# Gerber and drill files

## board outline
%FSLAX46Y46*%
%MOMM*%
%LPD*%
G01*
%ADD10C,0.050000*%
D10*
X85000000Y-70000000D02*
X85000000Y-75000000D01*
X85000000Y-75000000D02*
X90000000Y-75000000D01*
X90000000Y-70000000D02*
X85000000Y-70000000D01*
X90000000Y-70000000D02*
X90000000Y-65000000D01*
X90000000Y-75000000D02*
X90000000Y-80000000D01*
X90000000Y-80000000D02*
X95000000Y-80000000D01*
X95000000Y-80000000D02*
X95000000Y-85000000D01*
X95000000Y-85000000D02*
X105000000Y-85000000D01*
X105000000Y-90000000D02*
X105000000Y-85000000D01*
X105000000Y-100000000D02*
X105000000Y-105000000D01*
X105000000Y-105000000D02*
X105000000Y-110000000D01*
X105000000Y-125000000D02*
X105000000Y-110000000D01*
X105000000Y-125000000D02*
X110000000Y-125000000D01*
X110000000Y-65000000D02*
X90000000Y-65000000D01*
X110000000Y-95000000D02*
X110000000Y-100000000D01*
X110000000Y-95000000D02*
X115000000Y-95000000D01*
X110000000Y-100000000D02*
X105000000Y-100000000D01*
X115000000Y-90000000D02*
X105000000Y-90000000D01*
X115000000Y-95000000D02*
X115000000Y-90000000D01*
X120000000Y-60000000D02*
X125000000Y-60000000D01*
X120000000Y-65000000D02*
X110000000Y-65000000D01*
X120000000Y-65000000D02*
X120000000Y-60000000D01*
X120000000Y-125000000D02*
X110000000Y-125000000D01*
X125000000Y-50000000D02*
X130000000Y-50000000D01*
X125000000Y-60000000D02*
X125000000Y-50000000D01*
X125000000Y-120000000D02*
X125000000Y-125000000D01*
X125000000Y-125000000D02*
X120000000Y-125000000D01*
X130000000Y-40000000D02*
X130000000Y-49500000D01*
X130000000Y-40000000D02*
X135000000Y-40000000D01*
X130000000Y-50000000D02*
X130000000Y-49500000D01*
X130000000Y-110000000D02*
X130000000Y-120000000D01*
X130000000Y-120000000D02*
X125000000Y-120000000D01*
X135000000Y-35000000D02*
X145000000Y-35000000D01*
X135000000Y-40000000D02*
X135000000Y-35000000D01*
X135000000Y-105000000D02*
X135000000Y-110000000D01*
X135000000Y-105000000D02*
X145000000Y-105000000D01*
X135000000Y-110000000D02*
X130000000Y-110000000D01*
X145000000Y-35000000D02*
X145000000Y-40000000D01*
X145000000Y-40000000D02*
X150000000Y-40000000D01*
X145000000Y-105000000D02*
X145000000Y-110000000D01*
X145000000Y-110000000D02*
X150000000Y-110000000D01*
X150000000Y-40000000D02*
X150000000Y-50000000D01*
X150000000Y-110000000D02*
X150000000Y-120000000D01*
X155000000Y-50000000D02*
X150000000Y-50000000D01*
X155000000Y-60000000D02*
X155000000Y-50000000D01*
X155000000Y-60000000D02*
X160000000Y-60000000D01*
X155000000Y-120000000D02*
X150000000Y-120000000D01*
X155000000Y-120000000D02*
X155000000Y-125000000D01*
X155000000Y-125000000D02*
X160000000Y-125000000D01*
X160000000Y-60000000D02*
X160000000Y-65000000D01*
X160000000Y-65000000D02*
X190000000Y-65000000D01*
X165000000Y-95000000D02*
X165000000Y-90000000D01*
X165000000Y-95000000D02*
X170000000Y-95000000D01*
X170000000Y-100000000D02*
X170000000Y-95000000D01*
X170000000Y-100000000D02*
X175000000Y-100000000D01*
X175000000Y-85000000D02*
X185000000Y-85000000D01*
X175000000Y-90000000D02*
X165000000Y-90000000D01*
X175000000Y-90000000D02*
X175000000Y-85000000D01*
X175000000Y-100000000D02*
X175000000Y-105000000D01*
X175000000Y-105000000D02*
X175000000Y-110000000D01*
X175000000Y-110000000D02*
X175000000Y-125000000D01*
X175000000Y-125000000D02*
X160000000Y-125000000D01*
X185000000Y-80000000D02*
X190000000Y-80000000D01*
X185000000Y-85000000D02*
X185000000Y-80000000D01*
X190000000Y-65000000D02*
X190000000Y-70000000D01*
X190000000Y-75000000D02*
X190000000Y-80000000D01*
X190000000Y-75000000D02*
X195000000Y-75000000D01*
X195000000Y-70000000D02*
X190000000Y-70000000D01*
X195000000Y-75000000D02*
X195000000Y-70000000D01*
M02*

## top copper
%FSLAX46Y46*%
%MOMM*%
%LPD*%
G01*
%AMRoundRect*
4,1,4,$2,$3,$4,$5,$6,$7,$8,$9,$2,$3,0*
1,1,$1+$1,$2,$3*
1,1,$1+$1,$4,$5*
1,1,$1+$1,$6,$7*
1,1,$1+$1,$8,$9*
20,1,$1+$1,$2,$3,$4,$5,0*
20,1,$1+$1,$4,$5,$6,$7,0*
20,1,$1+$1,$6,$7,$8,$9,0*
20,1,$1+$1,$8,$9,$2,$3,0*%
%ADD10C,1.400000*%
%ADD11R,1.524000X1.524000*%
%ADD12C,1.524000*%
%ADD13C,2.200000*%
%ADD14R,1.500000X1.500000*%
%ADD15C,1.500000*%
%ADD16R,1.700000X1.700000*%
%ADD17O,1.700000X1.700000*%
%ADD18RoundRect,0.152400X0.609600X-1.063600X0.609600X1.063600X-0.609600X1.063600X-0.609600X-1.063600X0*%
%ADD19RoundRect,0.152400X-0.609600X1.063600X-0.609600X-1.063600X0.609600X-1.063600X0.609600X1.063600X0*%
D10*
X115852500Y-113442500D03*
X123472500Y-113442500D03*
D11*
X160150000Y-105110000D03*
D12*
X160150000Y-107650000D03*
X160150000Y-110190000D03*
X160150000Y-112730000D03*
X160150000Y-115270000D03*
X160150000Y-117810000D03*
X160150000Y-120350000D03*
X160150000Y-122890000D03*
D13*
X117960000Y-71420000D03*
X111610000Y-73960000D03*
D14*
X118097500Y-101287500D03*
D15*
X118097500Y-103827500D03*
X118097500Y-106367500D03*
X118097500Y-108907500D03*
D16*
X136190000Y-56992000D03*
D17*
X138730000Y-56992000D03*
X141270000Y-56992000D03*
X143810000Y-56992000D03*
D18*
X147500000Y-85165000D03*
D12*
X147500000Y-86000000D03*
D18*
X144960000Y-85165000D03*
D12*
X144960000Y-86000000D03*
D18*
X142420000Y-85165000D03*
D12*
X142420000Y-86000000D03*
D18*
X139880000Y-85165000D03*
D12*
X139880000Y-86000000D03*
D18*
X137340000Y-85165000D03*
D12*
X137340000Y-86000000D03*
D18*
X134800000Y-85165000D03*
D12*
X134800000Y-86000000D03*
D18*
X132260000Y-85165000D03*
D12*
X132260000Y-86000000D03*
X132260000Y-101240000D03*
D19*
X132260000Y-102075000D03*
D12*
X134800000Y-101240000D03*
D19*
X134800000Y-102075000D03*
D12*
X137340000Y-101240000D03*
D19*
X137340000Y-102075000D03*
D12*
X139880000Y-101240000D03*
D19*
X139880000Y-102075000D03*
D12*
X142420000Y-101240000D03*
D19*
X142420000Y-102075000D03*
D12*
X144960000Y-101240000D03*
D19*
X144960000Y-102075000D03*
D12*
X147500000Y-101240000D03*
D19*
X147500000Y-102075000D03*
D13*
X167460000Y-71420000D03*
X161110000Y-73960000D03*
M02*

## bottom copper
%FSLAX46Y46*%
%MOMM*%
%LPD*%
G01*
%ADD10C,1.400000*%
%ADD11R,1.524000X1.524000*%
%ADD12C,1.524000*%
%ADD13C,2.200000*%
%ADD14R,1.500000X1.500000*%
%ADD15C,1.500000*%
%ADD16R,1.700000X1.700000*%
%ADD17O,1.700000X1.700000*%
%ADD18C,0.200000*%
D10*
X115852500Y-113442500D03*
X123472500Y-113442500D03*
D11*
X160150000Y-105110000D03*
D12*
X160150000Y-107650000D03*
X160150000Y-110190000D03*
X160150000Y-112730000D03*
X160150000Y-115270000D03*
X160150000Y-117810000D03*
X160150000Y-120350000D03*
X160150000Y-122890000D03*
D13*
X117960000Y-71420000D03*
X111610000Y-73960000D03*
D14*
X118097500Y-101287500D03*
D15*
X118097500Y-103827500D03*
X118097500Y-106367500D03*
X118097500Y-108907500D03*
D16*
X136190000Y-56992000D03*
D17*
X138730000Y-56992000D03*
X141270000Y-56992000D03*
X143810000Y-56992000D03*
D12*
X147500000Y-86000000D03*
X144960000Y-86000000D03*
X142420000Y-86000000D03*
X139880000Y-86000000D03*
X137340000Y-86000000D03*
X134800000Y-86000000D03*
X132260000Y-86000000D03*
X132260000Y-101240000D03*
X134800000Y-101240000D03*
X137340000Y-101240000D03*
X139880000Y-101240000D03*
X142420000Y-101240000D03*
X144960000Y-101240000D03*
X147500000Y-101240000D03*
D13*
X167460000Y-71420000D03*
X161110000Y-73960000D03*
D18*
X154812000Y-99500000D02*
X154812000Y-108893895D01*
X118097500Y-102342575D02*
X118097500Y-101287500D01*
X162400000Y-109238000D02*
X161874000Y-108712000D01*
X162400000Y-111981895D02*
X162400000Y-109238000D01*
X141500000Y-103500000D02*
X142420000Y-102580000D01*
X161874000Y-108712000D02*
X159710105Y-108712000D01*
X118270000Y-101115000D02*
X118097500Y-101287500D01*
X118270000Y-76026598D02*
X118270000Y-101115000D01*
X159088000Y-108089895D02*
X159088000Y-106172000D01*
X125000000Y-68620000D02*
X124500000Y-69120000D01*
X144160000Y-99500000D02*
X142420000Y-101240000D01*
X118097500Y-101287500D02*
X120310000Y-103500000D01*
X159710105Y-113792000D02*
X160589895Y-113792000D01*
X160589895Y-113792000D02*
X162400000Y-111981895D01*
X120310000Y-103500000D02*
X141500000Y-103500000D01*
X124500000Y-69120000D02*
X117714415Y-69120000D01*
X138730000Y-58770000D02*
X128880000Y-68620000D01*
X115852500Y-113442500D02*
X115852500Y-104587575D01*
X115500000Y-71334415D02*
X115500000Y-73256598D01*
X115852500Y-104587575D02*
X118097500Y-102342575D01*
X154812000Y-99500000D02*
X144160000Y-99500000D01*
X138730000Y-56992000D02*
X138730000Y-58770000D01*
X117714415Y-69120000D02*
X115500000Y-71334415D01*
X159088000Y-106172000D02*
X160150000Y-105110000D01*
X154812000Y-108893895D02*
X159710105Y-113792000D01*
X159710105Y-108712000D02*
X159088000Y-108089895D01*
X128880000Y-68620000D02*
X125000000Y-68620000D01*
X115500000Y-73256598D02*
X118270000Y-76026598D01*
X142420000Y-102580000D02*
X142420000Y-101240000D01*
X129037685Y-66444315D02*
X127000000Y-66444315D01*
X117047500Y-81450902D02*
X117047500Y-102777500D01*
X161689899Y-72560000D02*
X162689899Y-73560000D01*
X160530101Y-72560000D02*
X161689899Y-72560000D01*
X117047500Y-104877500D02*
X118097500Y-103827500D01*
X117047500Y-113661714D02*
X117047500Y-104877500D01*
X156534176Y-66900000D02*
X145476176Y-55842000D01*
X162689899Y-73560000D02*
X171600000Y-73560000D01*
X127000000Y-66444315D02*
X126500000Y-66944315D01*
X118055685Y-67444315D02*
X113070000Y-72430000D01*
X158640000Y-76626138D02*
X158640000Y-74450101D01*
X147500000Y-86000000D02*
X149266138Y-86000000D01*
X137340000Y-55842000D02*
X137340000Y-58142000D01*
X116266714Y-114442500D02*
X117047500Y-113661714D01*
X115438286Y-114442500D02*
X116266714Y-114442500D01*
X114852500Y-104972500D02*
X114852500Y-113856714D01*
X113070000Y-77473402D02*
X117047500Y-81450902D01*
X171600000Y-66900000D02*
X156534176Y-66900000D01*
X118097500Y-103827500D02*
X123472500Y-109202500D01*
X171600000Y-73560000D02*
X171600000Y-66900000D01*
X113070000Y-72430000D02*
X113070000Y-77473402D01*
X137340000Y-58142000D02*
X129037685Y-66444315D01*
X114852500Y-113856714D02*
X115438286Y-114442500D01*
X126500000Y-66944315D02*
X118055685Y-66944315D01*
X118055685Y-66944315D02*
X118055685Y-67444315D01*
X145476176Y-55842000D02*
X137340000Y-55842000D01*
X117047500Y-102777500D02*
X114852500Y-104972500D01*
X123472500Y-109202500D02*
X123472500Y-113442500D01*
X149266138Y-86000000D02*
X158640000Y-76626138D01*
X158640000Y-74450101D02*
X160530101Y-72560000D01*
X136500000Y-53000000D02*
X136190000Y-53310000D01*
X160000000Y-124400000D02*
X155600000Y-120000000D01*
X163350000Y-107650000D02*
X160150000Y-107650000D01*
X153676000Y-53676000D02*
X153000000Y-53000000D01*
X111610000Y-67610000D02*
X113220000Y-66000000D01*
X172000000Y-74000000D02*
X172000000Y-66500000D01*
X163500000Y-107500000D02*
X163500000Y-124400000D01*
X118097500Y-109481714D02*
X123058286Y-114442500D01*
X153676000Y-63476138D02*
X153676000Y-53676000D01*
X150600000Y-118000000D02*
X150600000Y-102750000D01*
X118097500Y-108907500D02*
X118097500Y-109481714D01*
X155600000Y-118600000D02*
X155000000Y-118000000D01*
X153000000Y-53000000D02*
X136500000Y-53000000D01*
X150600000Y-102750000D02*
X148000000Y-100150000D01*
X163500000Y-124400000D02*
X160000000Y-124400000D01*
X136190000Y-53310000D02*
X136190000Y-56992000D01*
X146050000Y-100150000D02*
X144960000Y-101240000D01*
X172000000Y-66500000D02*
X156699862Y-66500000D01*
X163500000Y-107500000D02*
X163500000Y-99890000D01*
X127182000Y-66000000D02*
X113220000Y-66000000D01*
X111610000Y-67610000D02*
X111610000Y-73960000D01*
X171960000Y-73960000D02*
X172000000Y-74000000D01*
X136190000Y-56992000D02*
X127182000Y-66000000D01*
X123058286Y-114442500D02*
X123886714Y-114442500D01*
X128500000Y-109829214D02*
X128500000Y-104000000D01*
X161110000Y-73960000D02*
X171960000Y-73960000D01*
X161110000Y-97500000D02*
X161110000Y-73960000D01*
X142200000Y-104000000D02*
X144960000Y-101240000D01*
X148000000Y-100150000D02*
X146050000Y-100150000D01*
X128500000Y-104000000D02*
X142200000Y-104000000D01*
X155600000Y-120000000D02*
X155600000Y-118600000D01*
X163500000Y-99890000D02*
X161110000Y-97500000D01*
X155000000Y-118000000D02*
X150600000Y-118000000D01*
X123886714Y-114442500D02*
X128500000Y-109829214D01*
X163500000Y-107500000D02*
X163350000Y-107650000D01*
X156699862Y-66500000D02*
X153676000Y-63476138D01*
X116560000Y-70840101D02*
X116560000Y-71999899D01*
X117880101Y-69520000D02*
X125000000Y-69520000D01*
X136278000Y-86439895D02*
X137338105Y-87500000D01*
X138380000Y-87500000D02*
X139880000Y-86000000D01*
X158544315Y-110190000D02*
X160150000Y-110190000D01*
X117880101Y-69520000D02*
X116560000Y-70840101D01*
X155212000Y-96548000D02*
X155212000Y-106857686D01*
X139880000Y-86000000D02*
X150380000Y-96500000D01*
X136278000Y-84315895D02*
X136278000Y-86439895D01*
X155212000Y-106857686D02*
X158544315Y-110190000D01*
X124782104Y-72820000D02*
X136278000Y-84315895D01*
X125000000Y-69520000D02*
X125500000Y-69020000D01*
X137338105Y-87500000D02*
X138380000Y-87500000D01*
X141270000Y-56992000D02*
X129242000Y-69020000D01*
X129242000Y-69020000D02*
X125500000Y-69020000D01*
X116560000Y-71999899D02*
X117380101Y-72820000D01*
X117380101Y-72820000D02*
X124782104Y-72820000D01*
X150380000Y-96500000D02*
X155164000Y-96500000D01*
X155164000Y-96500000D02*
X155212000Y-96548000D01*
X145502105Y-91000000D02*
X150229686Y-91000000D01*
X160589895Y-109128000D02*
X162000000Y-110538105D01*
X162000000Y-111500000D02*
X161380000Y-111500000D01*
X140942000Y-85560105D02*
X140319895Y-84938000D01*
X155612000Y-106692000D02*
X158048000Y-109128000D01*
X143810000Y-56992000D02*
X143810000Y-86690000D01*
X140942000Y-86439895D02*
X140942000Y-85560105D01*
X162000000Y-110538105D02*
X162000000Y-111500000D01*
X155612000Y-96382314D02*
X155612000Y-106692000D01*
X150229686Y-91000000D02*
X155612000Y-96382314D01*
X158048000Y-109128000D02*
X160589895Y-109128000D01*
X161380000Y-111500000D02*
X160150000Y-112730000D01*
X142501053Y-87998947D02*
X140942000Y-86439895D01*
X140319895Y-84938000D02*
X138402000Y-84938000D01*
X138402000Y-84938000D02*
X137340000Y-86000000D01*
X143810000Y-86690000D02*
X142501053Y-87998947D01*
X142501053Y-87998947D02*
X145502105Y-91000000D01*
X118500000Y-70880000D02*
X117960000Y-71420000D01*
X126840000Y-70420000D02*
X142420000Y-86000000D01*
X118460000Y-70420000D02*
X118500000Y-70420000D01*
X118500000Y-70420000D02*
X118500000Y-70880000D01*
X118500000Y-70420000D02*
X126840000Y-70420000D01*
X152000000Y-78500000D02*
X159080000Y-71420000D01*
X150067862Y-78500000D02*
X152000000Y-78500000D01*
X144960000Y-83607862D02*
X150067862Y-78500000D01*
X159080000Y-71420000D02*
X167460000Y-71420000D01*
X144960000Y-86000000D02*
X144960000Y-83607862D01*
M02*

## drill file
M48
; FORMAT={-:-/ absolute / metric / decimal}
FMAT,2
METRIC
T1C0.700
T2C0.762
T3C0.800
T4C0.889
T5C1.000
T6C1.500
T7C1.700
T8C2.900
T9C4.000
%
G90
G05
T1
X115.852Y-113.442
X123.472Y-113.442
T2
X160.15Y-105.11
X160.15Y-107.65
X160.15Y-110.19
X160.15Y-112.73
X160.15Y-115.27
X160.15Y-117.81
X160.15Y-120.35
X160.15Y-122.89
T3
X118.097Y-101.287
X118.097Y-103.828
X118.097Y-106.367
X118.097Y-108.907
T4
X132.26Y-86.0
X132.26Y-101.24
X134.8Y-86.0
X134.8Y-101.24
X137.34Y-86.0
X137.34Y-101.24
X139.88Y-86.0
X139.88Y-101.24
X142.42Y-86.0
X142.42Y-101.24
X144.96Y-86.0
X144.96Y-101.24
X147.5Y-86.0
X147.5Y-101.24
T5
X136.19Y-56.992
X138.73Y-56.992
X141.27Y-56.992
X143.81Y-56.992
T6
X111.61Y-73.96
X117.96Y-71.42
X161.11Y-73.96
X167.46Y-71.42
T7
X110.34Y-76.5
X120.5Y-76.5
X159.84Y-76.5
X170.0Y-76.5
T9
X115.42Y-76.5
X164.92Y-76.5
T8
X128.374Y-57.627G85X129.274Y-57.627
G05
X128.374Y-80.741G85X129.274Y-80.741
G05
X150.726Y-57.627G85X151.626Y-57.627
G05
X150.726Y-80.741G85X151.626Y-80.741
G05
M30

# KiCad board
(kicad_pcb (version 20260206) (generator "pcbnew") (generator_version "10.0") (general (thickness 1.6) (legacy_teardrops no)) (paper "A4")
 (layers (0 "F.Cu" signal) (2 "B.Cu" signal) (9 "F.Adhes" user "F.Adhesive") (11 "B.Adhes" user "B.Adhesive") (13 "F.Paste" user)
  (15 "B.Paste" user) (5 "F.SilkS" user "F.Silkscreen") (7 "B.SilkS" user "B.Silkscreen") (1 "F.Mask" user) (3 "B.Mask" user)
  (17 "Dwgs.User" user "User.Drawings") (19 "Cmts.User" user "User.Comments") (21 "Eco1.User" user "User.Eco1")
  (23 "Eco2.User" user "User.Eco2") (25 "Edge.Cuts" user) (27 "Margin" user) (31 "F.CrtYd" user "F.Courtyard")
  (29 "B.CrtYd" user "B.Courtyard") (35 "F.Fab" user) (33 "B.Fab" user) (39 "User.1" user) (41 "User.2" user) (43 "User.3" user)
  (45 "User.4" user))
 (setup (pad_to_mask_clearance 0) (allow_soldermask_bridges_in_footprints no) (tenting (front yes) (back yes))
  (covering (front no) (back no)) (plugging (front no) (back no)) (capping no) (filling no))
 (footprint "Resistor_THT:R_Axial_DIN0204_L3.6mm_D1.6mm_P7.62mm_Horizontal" (layer "F.Cu") (at 115.8525 113.4425)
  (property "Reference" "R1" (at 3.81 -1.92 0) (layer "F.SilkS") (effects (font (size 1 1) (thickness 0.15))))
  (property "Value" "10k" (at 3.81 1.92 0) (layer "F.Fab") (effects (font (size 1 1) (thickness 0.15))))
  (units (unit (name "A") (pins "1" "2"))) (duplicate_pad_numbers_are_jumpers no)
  (pad "1" thru_hole circle (at 0 0) (size 1.4 1.4) (drill 0.7) (layers "*.Cu" "*.Mask") (remove_unused_layers no) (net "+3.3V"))
  (pad "2" thru_hole circle (at 7.62 0) (size 1.4 1.4) (drill 0.7) (layers "*.Cu" "*.Mask") (remove_unused_layers no) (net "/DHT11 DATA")))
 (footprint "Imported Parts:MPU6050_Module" (layer "F.Cu") (at 160.15 105.11)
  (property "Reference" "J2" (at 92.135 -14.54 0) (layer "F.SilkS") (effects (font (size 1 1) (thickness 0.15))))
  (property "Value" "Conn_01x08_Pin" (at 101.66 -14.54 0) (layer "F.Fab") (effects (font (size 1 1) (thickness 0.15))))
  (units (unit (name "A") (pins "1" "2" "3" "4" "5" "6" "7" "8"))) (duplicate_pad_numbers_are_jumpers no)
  (pad "1" thru_hole rect (at 0 0) (size 1.524 1.524) (drill 0.762) (layers "*.Cu" "*.Mask") (remove_unused_layers no) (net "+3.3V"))
  (pad "2" thru_hole circle (at 0 2.54) (size 1.524 1.524) (drill 0.762) (layers "*.Cu" "*.Mask") (remove_unused_layers no) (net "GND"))
  (pad "3" thru_hole circle (at 0 5.08) (size 1.524 1.524) (drill 0.762) (layers "*.Cu" "*.Mask") (remove_unused_layers no) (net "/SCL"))
  (pad "4" thru_hole circle (at 0 7.62) (size 1.524 1.524) (drill 0.762) (layers "*.Cu" "*.Mask") (remove_unused_layers no) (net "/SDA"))
  (pad "5" thru_hole circle (at 0 10.16) (size 1.524 1.524) (drill 0.762) (layers "*.Cu" "*.Mask") (remove_unused_layers no)
   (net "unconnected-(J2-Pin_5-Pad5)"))
  (pad "6" thru_hole circle (at 0 12.7) (size 1.524 1.524) (drill 0.762) (layers "*.Cu" "*.Mask") (remove_unused_layers no)
   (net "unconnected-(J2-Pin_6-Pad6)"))
  (pad "7" thru_hole circle (at 0 15.24) (size 1.524 1.524) (drill 0.762) (layers "*.Cu" "*.Mask") (remove_unused_layers no)
   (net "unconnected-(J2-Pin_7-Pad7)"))
  (pad "8" thru_hole circle (at 0 17.78) (size 1.524 1.524) (drill 0.762) (layers "*.Cu" "*.Mask") (remove_unused_layers no)
   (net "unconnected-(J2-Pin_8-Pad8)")))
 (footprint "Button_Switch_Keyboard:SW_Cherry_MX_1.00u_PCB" (layer "F.Cu") (at 117.96 71.42)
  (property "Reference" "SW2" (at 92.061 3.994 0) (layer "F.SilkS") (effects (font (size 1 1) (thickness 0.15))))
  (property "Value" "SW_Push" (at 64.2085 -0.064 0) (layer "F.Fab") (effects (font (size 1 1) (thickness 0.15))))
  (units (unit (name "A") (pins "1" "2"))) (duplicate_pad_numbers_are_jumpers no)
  (pad "" np_thru_hole circle (at -7.62 5.08) (size 1.7 1.7) (drill 1.7) (layers "*.Cu" "*.Mask"))
  (pad "" np_thru_hole circle (at -2.54 5.08) (size 4 4) (drill 4) (layers "*.Cu" "*.Mask"))
  (pad "" np_thru_hole circle (at 2.54 5.08) (size 1.7 1.7) (drill 1.7) (layers "*.Cu" "*.Mask"))
  (pad "1" thru_hole circle (at 0 0) (size 2.2 2.2) (drill 1.5) (layers "*.Cu" "*.Mask") (remove_unused_layers no) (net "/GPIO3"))
  (pad "2" thru_hole circle (at -6.35 2.54) (size 2.2 2.2) (drill 1.5) (layers "*.Cu" "*.Mask") (remove_unused_layers no) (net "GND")))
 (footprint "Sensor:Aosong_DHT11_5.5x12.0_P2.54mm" (layer "F.Cu") (at 118.0975 101.2875)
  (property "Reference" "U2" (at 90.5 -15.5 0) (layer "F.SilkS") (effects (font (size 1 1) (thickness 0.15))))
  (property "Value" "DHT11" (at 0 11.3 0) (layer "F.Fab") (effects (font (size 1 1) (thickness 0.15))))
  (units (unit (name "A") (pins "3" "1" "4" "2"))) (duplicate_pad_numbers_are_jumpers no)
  (pad "1" thru_hole rect (at 0 0) (size 1.5 1.5) (drill 0.8) (layers "*.Cu" "*.Mask") (remove_unused_layers no) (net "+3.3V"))
  (pad "2" thru_hole circle (at 0 2.54) (size 1.5 1.5) (drill 0.8) (layers "*.Cu" "*.Mask") (remove_unused_layers no) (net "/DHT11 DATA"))
  (pad "3" thru_hole circle (at 0 5.08) (size 1.5 1.5) (drill 0.8) (layers "*.Cu" "*.Mask") (remove_unused_layers no)
   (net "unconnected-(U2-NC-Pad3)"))
  (pad "4" thru_hole circle (at 0 7.62) (size 1.5 1.5) (drill 0.8) (layers "*.Cu" "*.Mask") (remove_unused_layers no) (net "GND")))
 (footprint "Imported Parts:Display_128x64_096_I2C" (layer "F.Cu") (at 140 56.992)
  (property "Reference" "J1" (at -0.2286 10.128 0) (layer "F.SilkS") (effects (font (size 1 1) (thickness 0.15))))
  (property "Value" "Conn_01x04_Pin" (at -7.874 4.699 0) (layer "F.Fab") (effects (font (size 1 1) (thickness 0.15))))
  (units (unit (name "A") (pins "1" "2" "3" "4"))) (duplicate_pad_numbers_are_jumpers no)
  (pad "" np_thru_hole oval (at -11.176 0.635) (size 3.8 2.9) (drill oval 3.8 2.9) (layers "*.Cu" "*.Mask"))
  (pad "" np_thru_hole oval (at -11.176 23.749) (size 3.8 2.9) (drill oval 3.8 2.9) (layers "*.Cu" "*.Mask"))
  (pad "" np_thru_hole oval (at 11.176 0.635) (size 3.8 2.9) (drill oval 3.8 2.9) (layers "*.Cu" "*.Mask"))
  (pad "" np_thru_hole oval (at 11.176 23.749) (size 3.8 2.9) (drill oval 3.8 2.9) (layers "*.Cu" "*.Mask"))
  (pad "1" thru_hole rect (at -3.81 0 90) (size 1.7 1.7) (drill 1) (layers "*.Cu" "*.Mask") (remove_unused_layers no) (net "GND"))
  (pad "2" thru_hole oval (at -1.27 0 90) (size 1.7 1.7) (drill 1) (layers "*.Cu" "*.Mask") (remove_unused_layers no) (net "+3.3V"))
  (pad "3" thru_hole oval (at 1.27 0 90) (size 1.7 1.7) (drill 1) (layers "*.Cu" "*.Mask") (remove_unused_layers no) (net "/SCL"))
  (pad "4" thru_hole oval (at 3.81 0 90) (size 1.7 1.7) (drill 1) (layers "*.Cu" "*.Mask") (remove_unused_layers no) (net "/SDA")))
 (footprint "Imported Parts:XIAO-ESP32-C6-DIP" (layer "F.Cu") (at 139.88 93.62)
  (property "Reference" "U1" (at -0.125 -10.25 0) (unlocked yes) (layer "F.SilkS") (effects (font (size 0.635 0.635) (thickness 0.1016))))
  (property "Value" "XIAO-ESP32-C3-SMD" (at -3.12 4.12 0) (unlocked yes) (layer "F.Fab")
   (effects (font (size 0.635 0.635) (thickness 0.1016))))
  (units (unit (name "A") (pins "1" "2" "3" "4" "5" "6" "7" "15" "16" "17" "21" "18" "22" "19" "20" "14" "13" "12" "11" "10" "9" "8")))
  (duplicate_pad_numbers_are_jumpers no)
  (pad "1" smd roundrect (at 7.62 -8.455 90) (size 2.432 1.524) (layers "F.Cu" "F.Mask") (roundrect_rratio 0.1) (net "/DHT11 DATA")
   (thermal_bridge_angle 45))
  (pad "1" thru_hole circle (at 7.62 -7.62 90) (size 1.524 1.524) (drill 0.889) (layers "*.Cu" "*.Mask") (remove_unused_layers no)
   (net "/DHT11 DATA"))
  (pad "2" smd roundrect (at 5.08 -8.455 90) (size 2.432 1.524) (layers "F.Cu" "F.Mask") (roundrect_rratio 0.1) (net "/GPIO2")
   (thermal_bridge_angle 45))
  (pad "2" thru_hole circle (at 5.08 -7.62 90) (size 1.524 1.524) (drill 0.889) (layers "*.Cu" "*.Mask") (remove_unused_layers no)
   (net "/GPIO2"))
  (pad "3" smd roundrect (at 2.54 -8.455 90) (size 2.432 1.524) (layers "F.Cu" "F.Mask") (roundrect_rratio 0.1) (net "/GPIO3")
   (thermal_bridge_angle 45))
  (pad "3" thru_hole circle (at 2.54 -7.62 90) (size 1.524 1.524) (drill 0.889) (layers "*.Cu" "*.Mask") (remove_unused_layers no)
   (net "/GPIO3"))
  (pad "4" smd roundrect (at 0 -8.455 90) (size 2.432 1.524) (layers "F.Cu" "F.Mask") (roundrect_rratio 0.1) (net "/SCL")
   (thermal_bridge_angle 45))
  (pad "4" thru_hole circle (at 0 -7.62 90) (size 1.524 1.524) (drill 0.889) (layers "*.Cu" "*.Mask") (remove_unused_layers no) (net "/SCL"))
  (pad "5" smd roundrect (at -2.54 -8.455 90) (size 2.432 1.524) (layers "F.Cu" "F.Mask") (roundrect_rratio 0.1) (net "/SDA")
   (thermal_bridge_angle 45))
  (pad "5" thru_hole circle (at -2.54 -7.62 90) (size 1.524 1.524) (drill 0.889) (layers "*.Cu" "*.Mask") (remove_unused_layers no)
   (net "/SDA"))
  (pad "6" smd roundrect (at -5.08 -8.455 90) (size 2.432 1.524) (layers "F.Cu" "F.Mask") (roundrect_rratio 0.1)
   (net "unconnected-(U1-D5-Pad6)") (thermal_bridge_angle 45))
  (pad "6" thru_hole circle (at -5.08 -7.62 90) (size 1.524 1.524) (drill 0.889) (layers "*.Cu" "*.Mask") (remove_unused_layers no)
   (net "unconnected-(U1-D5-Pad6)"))
  (pad "7" smd roundrect (at -7.62 -8.455 90) (size 2.432 1.524) (layers "F.Cu" "F.Mask") (roundrect_rratio 0.1)
   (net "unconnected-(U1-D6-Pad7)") (thermal_bridge_angle 45))
  (pad "7" thru_hole circle (at -7.62 -7.62 90) (size 1.524 1.524) (drill 0.889) (layers "*.Cu" "*.Mask") (remove_unused_layers no)
   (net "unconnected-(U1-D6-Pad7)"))
  (pad "8" thru_hole circle (at -7.62 7.62 270) (size 1.524 1.524) (drill 0.889) (layers "*.Cu" "*.Mask") (remove_unused_layers no)
   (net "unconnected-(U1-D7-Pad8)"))
  (pad "8" smd roundrect (at -7.62 8.455 270) (size 2.432 1.524) (layers "F.Cu" "F.Mask") (roundrect_rratio 0.1)
   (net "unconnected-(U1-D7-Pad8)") (thermal_bridge_angle 45))
  (pad "9" thru_hole circle (at -5.08 7.62 270) (size 1.524 1.524) (drill 0.889) (layers "*.Cu" "*.Mask") (remove_unused_layers no)
   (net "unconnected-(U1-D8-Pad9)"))
  (pad "9" smd roundrect (at -5.08 8.455 270) (size 2.432 1.524) (layers "F.Cu" "F.Mask") (roundrect_rratio 0.1)
   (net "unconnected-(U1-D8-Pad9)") (thermal_bridge_angle 45))
  (pad "10" thru_hole circle (at -2.54 7.62 270) (size 1.524 1.524) (drill 0.889) (layers "*.Cu" "*.Mask") (remove_unused_layers no)
   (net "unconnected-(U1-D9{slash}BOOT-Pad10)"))
  (pad "10" smd roundrect (at -2.54 8.455 270) (size 2.432 1.524) (layers "F.Cu" "F.Mask") (roundrect_rratio 0.1)
   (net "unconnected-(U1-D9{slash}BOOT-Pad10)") (thermal_bridge_angle 45))
  (pad "11" thru_hole circle (at 0 7.62 270) (size 1.524 1.524) (drill 0.889) (layers "*.Cu" "*.Mask") (remove_unused_layers no)
   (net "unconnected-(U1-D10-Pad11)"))
  (pad "11" smd roundrect (at 0 8.455 270) (size 2.432 1.524) (layers "F.Cu" "F.Mask") (roundrect_rratio 0.1)
   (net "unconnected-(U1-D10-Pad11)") (thermal_bridge_angle 45))
  (pad "12" thru_hole circle (at 2.54 7.62 270) (size 1.524 1.524) (drill 0.889) (layers "*.Cu" "*.Mask") (remove_unused_layers no)
   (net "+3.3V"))
  (pad "12" smd roundrect (at 2.54 8.455 270) (size 2.432 1.524) (layers "F.Cu" "F.Mask") (roundrect_rratio 0.1) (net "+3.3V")
   (thermal_bridge_angle 45))
  (pad "13" thru_hole circle (at 5.08 7.62 270) (size 1.524 1.524) (drill 0.889) (layers "*.Cu" "*.Mask") (remove_unused_layers no)
   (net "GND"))
  (pad "13" smd roundrect (at 5.08 8.455 270) (size 2.432 1.524) (layers "F.Cu" "F.Mask") (roundrect_rratio 0.1) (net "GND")
   (thermal_bridge_angle 45))
  (pad "14" thru_hole circle (at 7.62 7.62 270) (size 1.524 1.524) (drill 0.889) (layers "*.Cu" "*.Mask") (remove_unused_layers no)
   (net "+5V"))
  (pad "14" smd roundrect (at 7.62 8.455 270) (size 2.432 1.524) (layers "F.Cu" "F.Mask") (roundrect_rratio 0.1) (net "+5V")
   (thermal_bridge_angle 45)))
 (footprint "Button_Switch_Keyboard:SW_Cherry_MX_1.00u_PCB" (layer "F.Cu") (at 167.46 71.42)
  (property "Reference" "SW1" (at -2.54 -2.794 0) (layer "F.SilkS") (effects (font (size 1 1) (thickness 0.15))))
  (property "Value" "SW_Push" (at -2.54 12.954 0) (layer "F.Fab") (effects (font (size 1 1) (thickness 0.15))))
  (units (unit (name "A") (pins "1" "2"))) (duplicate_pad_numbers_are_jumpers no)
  (pad "" np_thru_hole circle (at -7.62 5.08) (size 1.7 1.7) (drill 1.7) (layers "*.Cu" "*.Mask"))
  (pad "" np_thru_hole circle (at -2.54 5.08) (size 4 4) (drill 4) (layers "*.Cu" "*.Mask"))
  (pad "" np_thru_hole circle (at 2.54 5.08) (size 1.7 1.7) (drill 1.7) (layers "*.Cu" "*.Mask"))
  (pad "1" thru_hole circle (at 0 0) (size 2.2 2.2) (drill 1.5) (layers "*.Cu" "*.Mask") (remove_unused_layers no) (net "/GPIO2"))
  (pad "2" thru_hole circle (at -6.35 2.54) (size 2.2 2.2) (drill 1.5) (layers "*.Cu" "*.Mask") (remove_unused_layers no) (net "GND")))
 (gr_line (start 85 70) (end 85 75) (stroke (width 0.05) (type default)) (layer "Edge.Cuts"))
 (gr_line (start 85 75) (end 90 75) (stroke (width 0.05) (type default)) (layer "Edge.Cuts"))
 (gr_line (start 90 70) (end 85 70) (stroke (width 0.05) (type default)) (layer "Edge.Cuts"))
 (gr_line (start 90 70) (end 90 65) (stroke (width 0.05) (type default)) (layer "Edge.Cuts"))
 (gr_line (start 90 75) (end 90 80) (stroke (width 0.05) (type default)) (layer "Edge.Cuts"))
 (gr_line (start 90 80) (end 95 80) (stroke (width 0.05) (type default)) (layer "Edge.Cuts"))
 (gr_line (start 95 80) (end 95 85) (stroke (width 0.05) (type default)) (layer "Edge.Cuts"))
 (gr_line (start 95 85) (end 105 85) (stroke (width 0.05) (type default)) (layer "Edge.Cuts"))
 (gr_line (start 105 90) (end 105 85) (stroke (width 0.05) (type default)) (layer "Edge.Cuts"))
 (gr_line (start 105 100) (end 105 105) (stroke (width 0.05) (type default)) (layer "Edge.Cuts"))
 (gr_line (start 105 105) (end 105 110) (stroke (width 0.05) (type default)) (layer "Edge.Cuts"))
 (gr_line (start 105 125) (end 105 110) (stroke (width 0.05) (type default)) (layer "Edge.Cuts"))
 (gr_line (start 105 125) (end 110 125) (stroke (width 0.05) (type default)) (layer "Edge.Cuts"))
 (gr_line (start 110 65) (end 90 65) (stroke (width 0.05) (type default)) (layer "Edge.Cuts"))
 (gr_line (start 110 95) (end 110 100) (stroke (width 0.05) (type default)) (layer "Edge.Cuts"))
 (gr_line (start 110 95) (end 115 95) (stroke (width 0.05) (type default)) (layer "Edge.Cuts"))
 (gr_line (start 110 100) (end 105 100) (stroke (width 0.05) (type default)) (layer "Edge.Cuts"))
 (gr_line (start 115 90) (end 105 90) (stroke (width 0.05) (type default)) (layer "Edge.Cuts"))
 (gr_line (start 115 95) (end 115 90) (stroke (width 0.05) (type default)) (layer "Edge.Cuts"))
 (gr_line (start 120 60) (end 125 60) (stroke (width 0.05) (type default)) (layer "Edge.Cuts"))
 (gr_line (start 120 65) (end 110 65) (stroke (width 0.05) (type default)) (layer "Edge.Cuts"))
 (gr_line (start 120 65) (end 120 60) (stroke (width 0.05) (type default)) (layer "Edge.Cuts"))
 (gr_line (start 120 125) (end 110 125) (stroke (width 0.05) (type default)) (layer "Edge.Cuts"))
 (gr_line (start 125 50) (end 130 50) (stroke (width 0.05) (type default)) (layer "Edge.Cuts"))
 (gr_line (start 125 60) (end 125 50) (stroke (width 0.05) (type default)) (layer "Edge.Cuts"))
 (gr_line (start 125 120) (end 125 125) (stroke (width 0.05) (type default)) (layer "Edge.Cuts"))
 (gr_line (start 125 125) (end 120 125) (stroke (width 0.05) (type default)) (layer "Edge.Cuts"))
 (gr_line (start 130 40) (end 130 49.5) (stroke (width 0.05) (type default)) (layer "Edge.Cuts"))
 (gr_line (start 130 40) (end 135 40) (stroke (width 0.05) (type default)) (layer "Edge.Cuts"))
 (gr_line (start 130 50) (end 130 49.5) (stroke (width 0.05) (type default)) (layer "Edge.Cuts"))
 (gr_line (start 130 110) (end 130 120) (stroke (width 0.05) (type default)) (layer "Edge.Cuts"))
 (gr_line (start 130 120) (end 125 120) (stroke (width 0.05) (type default)) (layer "Edge.Cuts"))
 (gr_line (start 135 35) (end 145 35) (stroke (width 0.05) (type default)) (layer "Edge.Cuts"))
 (gr_line (start 135 40) (end 135 35) (stroke (width 0.05) (type default)) (layer "Edge.Cuts"))
 (gr_line (start 135 105) (end 135 110) (stroke (width 0.05) (type default)) (layer "Edge.Cuts"))
 (gr_line (start 135 105) (end 145 105) (stroke (width 0.05) (type default)) (layer "Edge.Cuts"))
 (gr_line (start 135 110) (end 130 110) (stroke (width 0.05) (type default)) (layer "Edge.Cuts"))
 (gr_line (start 145 35) (end 145 40) (stroke (width 0.05) (type default)) (layer "Edge.Cuts"))
 (gr_line (start 145 40) (end 150 40) (stroke (width 0.05) (type default)) (layer "Edge.Cuts"))
 (gr_line (start 145 105) (end 145 110) (stroke (width 0.05) (type default)) (layer "Edge.Cuts"))
 (gr_line (start 145 110) (end 150 110) (stroke (width 0.05) (type default)) (layer "Edge.Cuts"))
 (gr_line (start 150 40) (end 150 50) (stroke (width 0.05) (type default)) (layer "Edge.Cuts"))
 (gr_line (start 150 110) (end 150 120) (stroke (width 0.05) (type default)) (layer "Edge.Cuts"))
 (gr_line (start 155 50) (end 150 50) (stroke (width 0.05) (type default)) (layer "Edge.Cuts"))
 (gr_line (start 155 60) (end 155 50) (stroke (width 0.05) (type default)) (layer "Edge.Cuts"))
 (gr_line (start 155 60) (end 160 60) (stroke (width 0.05) (type default)) (layer "Edge.Cuts"))
 (gr_line (start 155 120) (end 150 120) (stroke (width 0.05) (type default)) (layer "Edge.Cuts"))
 (gr_line (start 155 120) (end 155 125) (stroke (width 0.05) (type default)) (layer "Edge.Cuts"))
 (gr_line (start 155 125) (end 160 125) (stroke (width 0.05) (type default)) (layer "Edge.Cuts"))
 (gr_line (start 160 60) (end 160 65) (stroke (width 0.05) (type default)) (layer "Edge.Cuts"))
 (gr_line (start 160 65) (end 190 65) (stroke (width 0.05) (type default)) (layer "Edge.Cuts"))
 (gr_line (start 165 95) (end 165 90) (stroke (width 0.05) (type default)) (layer "Edge.Cuts"))
 (gr_line (start 165 95) (end 170 95) (stroke (width 0.05) (type default)) (layer "Edge.Cuts"))
 (gr_line (start 170 100) (end 170 95) (stroke (width 0.05) (type default)) (layer "Edge.Cuts"))
 (gr_line (start 170 100) (end 175 100) (stroke (width 0.05) (type default)) (layer "Edge.Cuts"))
 (gr_line (start 175 85) (end 185 85) (stroke (width 0.05) (type default)) (layer "Edge.Cuts"))
 (gr_line (start 175 90) (end 165 90) (stroke (width 0.05) (type default)) (layer "Edge.Cuts"))
 (gr_line (start 175 90) (end 175 85) (stroke (width 0.05) (type default)) (layer "Edge.Cuts"))
 (gr_line (start 175 100) (end 175 105) (stroke (width 0.05) (type default)) (layer "Edge.Cuts"))
 (gr_line (start 175 105) (end 175 110) (stroke (width 0.05) (type default)) (layer "Edge.Cuts"))
 (gr_line (start 175 110) (end 175 125) (stroke (width 0.05) (type default)) (layer "Edge.Cuts"))
 (gr_line (start 175 125) (end 160 125) (stroke (width 0.05) (type default)) (layer "Edge.Cuts"))
 (gr_line (start 185 80) (end 190 80) (stroke (width 0.05) (type default)) (layer "Edge.Cuts"))
 (gr_line (start 185 85) (end 185 80) (stroke (width 0.05) (type default)) (layer "Edge.Cuts"))
 (gr_line (start 190 65) (end 190 70) (stroke (width 0.05) (type default)) (layer "Edge.Cuts"))
 (gr_line (start 190 75) (end 190 80) (stroke (width 0.05) (type default)) (layer "Edge.Cuts"))
 (gr_line (start 190 75) (end 195 75) (stroke (width 0.05) (type default)) (layer "Edge.Cuts"))
 (gr_line (start 195 70) (end 190 70) (stroke (width 0.05) (type default)) (layer "Edge.Cuts"))
 (gr_line (start 195 75) (end 195 70) (stroke (width 0.05) (type default)) (layer "Edge.Cuts"))
 (segment (start 154.812 99.5) (end 154.812 108.893895) (width 0.2) (layer "B.Cu") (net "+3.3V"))
 (segment (start 118.0975 102.342575) (end 118.0975 101.2875) (width 0.2) (layer "B.Cu") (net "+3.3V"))
 (segment (start 162.4 109.238) (end 161.874 108.712) (width 0.2) (layer "B.Cu") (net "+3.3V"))
 (segment (start 162.4 111.981895) (end 162.4 109.238) (width 0.2) (layer "B.Cu") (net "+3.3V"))
 (segment (start 141.5 103.5) (end 142.42 102.58) (width 0.2) (layer "B.Cu") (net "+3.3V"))
 (segment (start 161.874 108.712) (end 159.710105 108.712) (width 0.2) (layer "B.Cu") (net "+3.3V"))
 (segment (start 118.27 101.115) (end 118.0975 101.2875) (width 0.2) (layer "B.Cu") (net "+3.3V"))
 (segment (start 118.27 76.026598) (end 118.27 101.115) (width 0.2) (layer "B.Cu") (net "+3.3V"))
 (segment (start 159.088 108.089895) (end 159.088 106.172) (width 0.2) (layer "B.Cu") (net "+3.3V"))
 (segment (start 125 68.62) (end 124.5 69.12) (width 0.2) (layer "B.Cu") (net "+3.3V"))
 (segment (start 144.16 99.5) (end 142.42 101.24) (width 0.2) (layer "B.Cu") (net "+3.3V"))
 (segment (start 118.0975 101.2875) (end 120.31 103.5) (width 0.2) (layer "B.Cu") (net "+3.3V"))
 (segment (start 159.710105 113.792) (end 160.589895 113.792) (width 0.2) (layer "B.Cu") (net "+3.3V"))
 (segment (start 160.589895 113.792) (end 162.4 111.981895) (width 0.2) (layer "B.Cu") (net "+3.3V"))
 (segment (start 120.31 103.5) (end 141.5 103.5) (width 0.2) (layer "B.Cu") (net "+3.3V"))
 (segment (start 124.5 69.12) (end 117.714415 69.12) (width 0.2) (layer "B.Cu") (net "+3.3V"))
 (segment (start 138.73 58.77) (end 128.88 68.62) (width 0.2) (layer "B.Cu") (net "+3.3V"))
 (segment (start 115.8525 113.4425) (end 115.8525 104.587575) (width 0.2) (layer "B.Cu") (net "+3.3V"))
 (segment (start 115.5 71.334415) (end 115.5 73.256598) (width 0.2) (layer "B.Cu") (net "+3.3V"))
 (segment (start 115.8525 104.587575) (end 118.0975 102.342575) (width 0.2) (layer "B.Cu") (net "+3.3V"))
 (segment (start 154.812 99.5) (end 144.16 99.5) (width 0.2) (layer "B.Cu") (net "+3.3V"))
 (segment (start 138.73 56.992) (end 138.73 58.77) (width 0.2) (layer "B.Cu") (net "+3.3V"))
 (segment (start 117.714415 69.12) (end 115.5 71.334415) (width 0.2) (layer "B.Cu") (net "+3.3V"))
 (segment (start 159.088 106.172) (end 160.15 105.11) (width 0.2) (layer "B.Cu") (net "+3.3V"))
 (segment (start 154.812 108.893895) (end 159.710105 113.792) (width 0.2) (layer "B.Cu") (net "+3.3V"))
 (segment (start 159.710105 108.712) (end 159.088 108.089895) (width 0.2) (layer "B.Cu") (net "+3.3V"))
 (segment (start 128.88 68.62) (end 125 68.62) (width 0.2) (layer "B.Cu") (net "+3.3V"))
 (segment (start 115.5 73.256598) (end 118.27 76.026598) (width 0.2) (layer "B.Cu") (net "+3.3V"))
 (segment (start 142.42 102.58) (end 142.42 101.24) (width 0.2) (layer "B.Cu") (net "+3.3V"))
 (segment (start 129.037685 66.444315) (end 127 66.444315) (width 0.2) (layer "B.Cu") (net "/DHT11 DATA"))
 (segment (start 117.0475 81.450902) (end 117.0475 102.7775) (width 0.2) (layer "B.Cu") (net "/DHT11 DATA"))
 (segment (start 161.689899 72.56) (end 162.689899 73.56) (width 0.2) (layer "B.Cu") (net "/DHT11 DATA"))
 (segment (start 160.530101 72.56) (end 161.689899 72.56) (width 0.2) (layer "B.Cu") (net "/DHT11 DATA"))
 (segment (start 117.0475 104.8775) (end 118.0975 103.8275) (width 0.2) (layer "B.Cu") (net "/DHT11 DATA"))
 (segment (start 117.0475 113.661714) (end 117.0475 104.8775) (width 0.2) (layer "B.Cu") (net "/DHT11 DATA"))
 (segment (start 156.534176 66.9) (end 145.476176 55.842) (width 0.2) (layer "B.Cu") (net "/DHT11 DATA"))
 (segment (start 162.689899 73.56) (end 171.6 73.56) (width 0.2) (layer "B.Cu") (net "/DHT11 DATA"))
 (segment (start 127 66.444315) (end 126.5 66.944315) (width 0.2) (layer "B.Cu") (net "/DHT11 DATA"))
 (segment (start 118.055685 67.444315) (end 113.07 72.43) (width 0.2) (layer "B.Cu") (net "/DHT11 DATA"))
 (segment (start 158.64 76.626138) (end 158.64 74.450101) (width 0.2) (layer "B.Cu") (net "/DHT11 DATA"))
 (segment (start 147.5 86) (end 149.266138 86) (width 0.2) (layer "B.Cu") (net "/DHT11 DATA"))
 (segment (start 137.34 55.842) (end 137.34 58.142) (width 0.2) (layer "B.Cu") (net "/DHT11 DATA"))
 (segment (start 116.266714 114.4425) (end 117.0475 113.661714) (width 0.2) (layer "B.Cu") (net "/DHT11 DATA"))
 (segment (start 115.438286 114.4425) (end 116.266714 114.4425) (width 0.2) (layer "B.Cu") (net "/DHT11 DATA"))
 (segment (start 114.8525 104.9725) (end 114.8525 113.856714) (width 0.2) (layer "B.Cu") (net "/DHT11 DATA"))
 (segment (start 113.07 77.473402) (end 117.0475 81.450902) (width 0.2) (layer "B.Cu") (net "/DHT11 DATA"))
 (segment (start 171.6 66.9) (end 156.534176 66.9) (width 0.2) (layer "B.Cu") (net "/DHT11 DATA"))
 (segment (start 118.0975 103.8275) (end 123.4725 109.2025) (width 0.2) (layer "B.Cu") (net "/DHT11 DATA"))
 (segment (start 171.6 73.56) (end 171.6 66.9) (width 0.2) (layer "B.Cu") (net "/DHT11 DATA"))
 (segment (start 113.07 72.43) (end 113.07 77.473402) (width 0.2) (layer "B.Cu") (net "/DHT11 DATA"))
 (segment (start 137.34 58.142) (end 129.037685 66.444315) (width 0.2) (layer "B.Cu") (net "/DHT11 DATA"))
 (segment (start 114.8525 113.856714) (end 115.438286 114.4425) (width 0.2) (layer "B.Cu") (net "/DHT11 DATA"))
 (segment (start 126.5 66.944315) (end 118.055685 66.944315) (width 0.2) (layer "B.Cu") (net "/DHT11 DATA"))
 (segment (start 118.055685 66.944315) (end 118.055685 67.444315) (width 0.2) (layer "B.Cu") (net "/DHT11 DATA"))
 (segment (start 145.476176 55.842) (end 137.34 55.842) (width 0.2) (layer "B.Cu") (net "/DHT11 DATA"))
 (segment (start 117.0475 102.7775) (end 114.8525 104.9725) (width 0.2) (layer "B.Cu") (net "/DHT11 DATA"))
 (segment (start 123.4725 109.2025) (end 123.4725 113.4425) (width 0.2) (layer "B.Cu") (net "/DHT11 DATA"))
 (segment (start 149.266138 86) (end 158.64 76.626138) (width 0.2) (layer "B.Cu") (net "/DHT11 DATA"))
 (segment (start 158.64 74.450101) (end 160.530101 72.56) (width 0.2) (layer "B.Cu") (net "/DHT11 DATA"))
 (segment (start 136.5 53) (end 136.19 53.31) (width 0.2) (layer "B.Cu") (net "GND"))
 (segment (start 160 124.4) (end 155.6 120) (width 0.2) (layer "B.Cu") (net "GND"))
 (segment (start 163.35 107.65) (end 160.15 107.65) (width 0.2) (layer "B.Cu") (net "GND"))
 (segment (start 153.676 53.676) (end 153 53) (width 0.2) (layer "B.Cu") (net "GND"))
 (segment (start 111.61 67.61) (end 113.22 66) (width 0.2) (layer "B.Cu") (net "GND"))
 (segment (start 172 74) (end 172 66.5) (width 0.2) (layer "B.Cu") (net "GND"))
 (segment (start 163.5 107.5) (end 163.5 124.4) (width 0.2) (layer "B.Cu") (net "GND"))
 (segment (start 118.0975 109.481714) (end 123.058286 114.4425) (width 0.2) (layer "B.Cu") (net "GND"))
 (segment (start 153.676 63.476138) (end 153.676 53.676) (width 0.2) (layer "B.Cu") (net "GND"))
 (segment (start 150.6 118) (end 150.6 102.75) (width 0.2) (layer "B.Cu") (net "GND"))
 (segment (start 118.0975 108.9075) (end 118.0975 109.481714) (width 0.2) (layer "B.Cu") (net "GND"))
 (segment (start 155.6 118.6) (end 155 118) (width 0.2) (layer "B.Cu") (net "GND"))
 (segment (start 153 53) (end 136.5 53) (width 0.2) (layer "B.Cu") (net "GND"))
 (segment (start 150.6 102.75) (end 148 100.15) (width 0.2) (layer "B.Cu") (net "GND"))
 (segment (start 163.5 124.4) (end 160 124.4) (width 0.2) (layer "B.Cu") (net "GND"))
 (segment (start 136.19 53.31) (end 136.19 56.992) (width 0.2) (layer "B.Cu") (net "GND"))
 (segment (start 146.05 100.15) (end 144.96 101.24) (width 0.2) (layer "B.Cu") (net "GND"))
 (segment (start 172 66.5) (end 156.699862 66.5) (width 0.2) (layer "B.Cu") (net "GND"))
 (segment (start 163.5 107.5) (end 163.5 99.89) (width 0.2) (layer "B.Cu") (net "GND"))
 (segment (start 127.182 66) (end 113.22 66) (width 0.2) (layer "B.Cu") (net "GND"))
 (segment (start 111.61 67.61) (end 111.61 73.96) (width 0.2) (layer "B.Cu") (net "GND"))
 (segment (start 171.96 73.96) (end 172 74) (width 0.2) (layer "B.Cu") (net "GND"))
 (segment (start 136.19 56.992) (end 127.182 66) (width 0.2) (layer "B.Cu") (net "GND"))
 (segment (start 123.058286 114.4425) (end 123.886714 114.4425) (width 0.2) (layer "B.Cu") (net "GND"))
 (segment (start 128.5 109.829214) (end 128.5 104) (width 0.2) (layer "B.Cu") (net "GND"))
 (segment (start 161.11 73.96) (end 171.96 73.96) (width 0.2) (layer "B.Cu") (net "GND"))
 (segment (start 161.11 97.5) (end 161.11 73.96) (width 0.2) (layer "B.Cu") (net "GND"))
 (segment (start 142.2 104) (end 144.96 101.24) (width 0.2) (layer "B.Cu") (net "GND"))
 (segment (start 148 100.15) (end 146.05 100.15) (width 0.2) (layer "B.Cu") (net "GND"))
 (segment (start 128.5 104) (end 142.2 104) (width 0.2) (layer "B.Cu") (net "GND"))
 (segment (start 155.6 120) (end 155.6 118.6) (width 0.2) (layer "B.Cu") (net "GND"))
 (segment (start 163.5 99.89) (end 161.11 97.5) (width 0.2) (layer "B.Cu") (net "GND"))
 (segment (start 155 118) (end 150.6 118) (width 0.2) (layer "B.Cu") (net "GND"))
 (segment (start 123.886714 114.4425) (end 128.5 109.829214) (width 0.2) (layer "B.Cu") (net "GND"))
 (segment (start 163.5 107.5) (end 163.35 107.65) (width 0.2) (layer "B.Cu") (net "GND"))
 (segment (start 156.699862 66.5) (end 153.676 63.476138) (width 0.2) (layer "B.Cu") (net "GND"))
 (segment (start 116.56 70.840101) (end 116.56 71.999899) (width 0.2) (layer "B.Cu") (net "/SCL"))
 (segment (start 117.880101 69.52) (end 125 69.52) (width 0.2) (layer "B.Cu") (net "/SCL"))
 (segment (start 136.278 86.439895) (end 137.338105 87.5) (width 0.2) (layer "B.Cu") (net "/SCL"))
 (segment (start 138.38 87.5) (end 139.88 86) (width 0.2) (layer "B.Cu") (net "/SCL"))
 (segment (start 158.544315 110.19) (end 160.15 110.19) (width 0.2) (layer "B.Cu") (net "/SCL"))
 (segment (start 117.880101 69.52) (end 116.56 70.840101) (width 0.2) (layer "B.Cu") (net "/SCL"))
 (segment (start 155.212 96.548) (end 155.212 106.857686) (width 0.2) (layer "B.Cu") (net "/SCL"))
 (segment (start 139.88 86) (end 150.38 96.5) (width 0.2) (layer "B.Cu") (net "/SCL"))
 (segment (start 136.278 84.315895) (end 136.278 86.439895) (width 0.2) (layer "B.Cu") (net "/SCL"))
 (segment (start 155.212 106.857686) (end 158.544315 110.19) (width 0.2) (layer "B.Cu") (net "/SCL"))
 (segment (start 124.782104 72.82) (end 136.278 84.315895) (width 0.2) (layer "B.Cu") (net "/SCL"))
 (segment (start 125 69.52) (end 125.5 69.02) (width 0.2) (layer "B.Cu") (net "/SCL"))
 (segment (start 137.338105 87.5) (end 138.38 87.5) (width 0.2) (layer "B.Cu") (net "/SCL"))
 (segment (start 141.27 56.992) (end 129.242 69.02) (width 0.2) (layer "B.Cu") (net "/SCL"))
 (segment (start 129.242 69.02) (end 125.5 69.02) (width 0.2) (layer "B.Cu") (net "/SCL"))
 (segment (start 116.56 71.999899) (end 117.380101 72.82) (width 0.2) (layer "B.Cu") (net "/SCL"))
 (segment (start 117.380101 72.82) (end 124.782104 72.82) (width 0.2) (layer "B.Cu") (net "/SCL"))
 (segment (start 150.38 96.5) (end 155.164 96.5) (width 0.2) (layer "B.Cu") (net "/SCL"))
 (segment (start 155.164 96.5) (end 155.212 96.548) (width 0.2) (layer "B.Cu") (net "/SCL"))
 (segment (start 145.502105 91) (end 150.229686 91) (width 0.2) (layer "B.Cu") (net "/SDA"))
 (segment (start 160.589895 109.128) (end 162 110.538105) (width 0.2) (layer "B.Cu") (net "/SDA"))
 (segment (start 162 111.5) (end 161.38 111.5) (width 0.2) (layer "B.Cu") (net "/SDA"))
 (segment (start 140.942 85.560105) (end 140.319895 84.938) (width 0.2) (layer "B.Cu") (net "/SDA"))
 (segment (start 155.612 106.692) (end 158.048 109.128) (width 0.2) (layer "B.Cu") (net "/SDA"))
 (segment (start 143.81 56.992) (end 143.81 86.69) (width 0.2) (layer "B.Cu") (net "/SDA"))
 (segment (start 140.942 86.439895) (end 140.942 85.560105) (width 0.2) (layer "B.Cu") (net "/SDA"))
 (segment (start 162 110.538105) (end 162 111.5) (width 0.2) (layer "B.Cu") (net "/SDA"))
 (segment (start 155.612 96.382314) (end 155.612 106.692) (width 0.2) (layer "B.Cu") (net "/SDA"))
 (segment (start 150.229686 91) (end 155.612 96.382314) (width 0.2) (layer "B.Cu") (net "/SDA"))
 (segment (start 158.048 109.128) (end 160.589895 109.128) (width 0.2) (layer "B.Cu") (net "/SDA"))
 (segment (start 161.38 111.5) (end 160.15 112.73) (width 0.2) (layer "B.Cu") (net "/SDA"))
 (segment (start 142.501053 87.998947) (end 140.942 86.439895) (width 0.2) (layer "B.Cu") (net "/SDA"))
 (segment (start 140.319895 84.938) (end 138.402 84.938) (width 0.2) (layer "B.Cu") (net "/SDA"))
 (segment (start 138.402 84.938) (end 137.34 86) (width 0.2) (layer "B.Cu") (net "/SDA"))
 (segment (start 143.81 86.69) (end 142.501053 87.998947) (width 0.2) (layer "B.Cu") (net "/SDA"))
 (segment (start 142.501053 87.998947) (end 145.502105 91) (width 0.2) (layer "B.Cu") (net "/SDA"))
 (segment (start 118.5 70.88) (end 117.96 71.42) (width 0.2) (layer "B.Cu") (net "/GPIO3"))
 (segment (start 126.84 70.42) (end 142.42 86) (width 0.2) (layer "B.Cu") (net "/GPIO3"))
 (segment (start 118.46 70.42) (end 118.5 70.42) (width 0.2) (layer "B.Cu") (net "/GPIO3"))
 (segment (start 118.5 70.42) (end 118.5 70.88) (width 0.2) (layer "B.Cu") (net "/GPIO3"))
 (segment (start 118.5 70.42) (end 126.84 70.42) (width 0.2) (layer "B.Cu") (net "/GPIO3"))
 (segment (start 152 78.5) (end 159.08 71.42) (width 0.2) (layer "B.Cu") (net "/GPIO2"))
 (segment (start 150.067862 78.5) (end 152 78.5) (width 0.2) (layer "B.Cu") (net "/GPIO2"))
 (segment (start 144.96 83.607862) (end 150.067862 78.5) (width 0.2) (layer "B.Cu") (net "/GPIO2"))
 (segment (start 159.08 71.42) (end 167.46 71.42) (width 0.2) (layer "B.Cu") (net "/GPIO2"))
 (segment (start 144.96 86) (end 144.96 83.607862) (width 0.2) (layer "B.Cu") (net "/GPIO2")))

